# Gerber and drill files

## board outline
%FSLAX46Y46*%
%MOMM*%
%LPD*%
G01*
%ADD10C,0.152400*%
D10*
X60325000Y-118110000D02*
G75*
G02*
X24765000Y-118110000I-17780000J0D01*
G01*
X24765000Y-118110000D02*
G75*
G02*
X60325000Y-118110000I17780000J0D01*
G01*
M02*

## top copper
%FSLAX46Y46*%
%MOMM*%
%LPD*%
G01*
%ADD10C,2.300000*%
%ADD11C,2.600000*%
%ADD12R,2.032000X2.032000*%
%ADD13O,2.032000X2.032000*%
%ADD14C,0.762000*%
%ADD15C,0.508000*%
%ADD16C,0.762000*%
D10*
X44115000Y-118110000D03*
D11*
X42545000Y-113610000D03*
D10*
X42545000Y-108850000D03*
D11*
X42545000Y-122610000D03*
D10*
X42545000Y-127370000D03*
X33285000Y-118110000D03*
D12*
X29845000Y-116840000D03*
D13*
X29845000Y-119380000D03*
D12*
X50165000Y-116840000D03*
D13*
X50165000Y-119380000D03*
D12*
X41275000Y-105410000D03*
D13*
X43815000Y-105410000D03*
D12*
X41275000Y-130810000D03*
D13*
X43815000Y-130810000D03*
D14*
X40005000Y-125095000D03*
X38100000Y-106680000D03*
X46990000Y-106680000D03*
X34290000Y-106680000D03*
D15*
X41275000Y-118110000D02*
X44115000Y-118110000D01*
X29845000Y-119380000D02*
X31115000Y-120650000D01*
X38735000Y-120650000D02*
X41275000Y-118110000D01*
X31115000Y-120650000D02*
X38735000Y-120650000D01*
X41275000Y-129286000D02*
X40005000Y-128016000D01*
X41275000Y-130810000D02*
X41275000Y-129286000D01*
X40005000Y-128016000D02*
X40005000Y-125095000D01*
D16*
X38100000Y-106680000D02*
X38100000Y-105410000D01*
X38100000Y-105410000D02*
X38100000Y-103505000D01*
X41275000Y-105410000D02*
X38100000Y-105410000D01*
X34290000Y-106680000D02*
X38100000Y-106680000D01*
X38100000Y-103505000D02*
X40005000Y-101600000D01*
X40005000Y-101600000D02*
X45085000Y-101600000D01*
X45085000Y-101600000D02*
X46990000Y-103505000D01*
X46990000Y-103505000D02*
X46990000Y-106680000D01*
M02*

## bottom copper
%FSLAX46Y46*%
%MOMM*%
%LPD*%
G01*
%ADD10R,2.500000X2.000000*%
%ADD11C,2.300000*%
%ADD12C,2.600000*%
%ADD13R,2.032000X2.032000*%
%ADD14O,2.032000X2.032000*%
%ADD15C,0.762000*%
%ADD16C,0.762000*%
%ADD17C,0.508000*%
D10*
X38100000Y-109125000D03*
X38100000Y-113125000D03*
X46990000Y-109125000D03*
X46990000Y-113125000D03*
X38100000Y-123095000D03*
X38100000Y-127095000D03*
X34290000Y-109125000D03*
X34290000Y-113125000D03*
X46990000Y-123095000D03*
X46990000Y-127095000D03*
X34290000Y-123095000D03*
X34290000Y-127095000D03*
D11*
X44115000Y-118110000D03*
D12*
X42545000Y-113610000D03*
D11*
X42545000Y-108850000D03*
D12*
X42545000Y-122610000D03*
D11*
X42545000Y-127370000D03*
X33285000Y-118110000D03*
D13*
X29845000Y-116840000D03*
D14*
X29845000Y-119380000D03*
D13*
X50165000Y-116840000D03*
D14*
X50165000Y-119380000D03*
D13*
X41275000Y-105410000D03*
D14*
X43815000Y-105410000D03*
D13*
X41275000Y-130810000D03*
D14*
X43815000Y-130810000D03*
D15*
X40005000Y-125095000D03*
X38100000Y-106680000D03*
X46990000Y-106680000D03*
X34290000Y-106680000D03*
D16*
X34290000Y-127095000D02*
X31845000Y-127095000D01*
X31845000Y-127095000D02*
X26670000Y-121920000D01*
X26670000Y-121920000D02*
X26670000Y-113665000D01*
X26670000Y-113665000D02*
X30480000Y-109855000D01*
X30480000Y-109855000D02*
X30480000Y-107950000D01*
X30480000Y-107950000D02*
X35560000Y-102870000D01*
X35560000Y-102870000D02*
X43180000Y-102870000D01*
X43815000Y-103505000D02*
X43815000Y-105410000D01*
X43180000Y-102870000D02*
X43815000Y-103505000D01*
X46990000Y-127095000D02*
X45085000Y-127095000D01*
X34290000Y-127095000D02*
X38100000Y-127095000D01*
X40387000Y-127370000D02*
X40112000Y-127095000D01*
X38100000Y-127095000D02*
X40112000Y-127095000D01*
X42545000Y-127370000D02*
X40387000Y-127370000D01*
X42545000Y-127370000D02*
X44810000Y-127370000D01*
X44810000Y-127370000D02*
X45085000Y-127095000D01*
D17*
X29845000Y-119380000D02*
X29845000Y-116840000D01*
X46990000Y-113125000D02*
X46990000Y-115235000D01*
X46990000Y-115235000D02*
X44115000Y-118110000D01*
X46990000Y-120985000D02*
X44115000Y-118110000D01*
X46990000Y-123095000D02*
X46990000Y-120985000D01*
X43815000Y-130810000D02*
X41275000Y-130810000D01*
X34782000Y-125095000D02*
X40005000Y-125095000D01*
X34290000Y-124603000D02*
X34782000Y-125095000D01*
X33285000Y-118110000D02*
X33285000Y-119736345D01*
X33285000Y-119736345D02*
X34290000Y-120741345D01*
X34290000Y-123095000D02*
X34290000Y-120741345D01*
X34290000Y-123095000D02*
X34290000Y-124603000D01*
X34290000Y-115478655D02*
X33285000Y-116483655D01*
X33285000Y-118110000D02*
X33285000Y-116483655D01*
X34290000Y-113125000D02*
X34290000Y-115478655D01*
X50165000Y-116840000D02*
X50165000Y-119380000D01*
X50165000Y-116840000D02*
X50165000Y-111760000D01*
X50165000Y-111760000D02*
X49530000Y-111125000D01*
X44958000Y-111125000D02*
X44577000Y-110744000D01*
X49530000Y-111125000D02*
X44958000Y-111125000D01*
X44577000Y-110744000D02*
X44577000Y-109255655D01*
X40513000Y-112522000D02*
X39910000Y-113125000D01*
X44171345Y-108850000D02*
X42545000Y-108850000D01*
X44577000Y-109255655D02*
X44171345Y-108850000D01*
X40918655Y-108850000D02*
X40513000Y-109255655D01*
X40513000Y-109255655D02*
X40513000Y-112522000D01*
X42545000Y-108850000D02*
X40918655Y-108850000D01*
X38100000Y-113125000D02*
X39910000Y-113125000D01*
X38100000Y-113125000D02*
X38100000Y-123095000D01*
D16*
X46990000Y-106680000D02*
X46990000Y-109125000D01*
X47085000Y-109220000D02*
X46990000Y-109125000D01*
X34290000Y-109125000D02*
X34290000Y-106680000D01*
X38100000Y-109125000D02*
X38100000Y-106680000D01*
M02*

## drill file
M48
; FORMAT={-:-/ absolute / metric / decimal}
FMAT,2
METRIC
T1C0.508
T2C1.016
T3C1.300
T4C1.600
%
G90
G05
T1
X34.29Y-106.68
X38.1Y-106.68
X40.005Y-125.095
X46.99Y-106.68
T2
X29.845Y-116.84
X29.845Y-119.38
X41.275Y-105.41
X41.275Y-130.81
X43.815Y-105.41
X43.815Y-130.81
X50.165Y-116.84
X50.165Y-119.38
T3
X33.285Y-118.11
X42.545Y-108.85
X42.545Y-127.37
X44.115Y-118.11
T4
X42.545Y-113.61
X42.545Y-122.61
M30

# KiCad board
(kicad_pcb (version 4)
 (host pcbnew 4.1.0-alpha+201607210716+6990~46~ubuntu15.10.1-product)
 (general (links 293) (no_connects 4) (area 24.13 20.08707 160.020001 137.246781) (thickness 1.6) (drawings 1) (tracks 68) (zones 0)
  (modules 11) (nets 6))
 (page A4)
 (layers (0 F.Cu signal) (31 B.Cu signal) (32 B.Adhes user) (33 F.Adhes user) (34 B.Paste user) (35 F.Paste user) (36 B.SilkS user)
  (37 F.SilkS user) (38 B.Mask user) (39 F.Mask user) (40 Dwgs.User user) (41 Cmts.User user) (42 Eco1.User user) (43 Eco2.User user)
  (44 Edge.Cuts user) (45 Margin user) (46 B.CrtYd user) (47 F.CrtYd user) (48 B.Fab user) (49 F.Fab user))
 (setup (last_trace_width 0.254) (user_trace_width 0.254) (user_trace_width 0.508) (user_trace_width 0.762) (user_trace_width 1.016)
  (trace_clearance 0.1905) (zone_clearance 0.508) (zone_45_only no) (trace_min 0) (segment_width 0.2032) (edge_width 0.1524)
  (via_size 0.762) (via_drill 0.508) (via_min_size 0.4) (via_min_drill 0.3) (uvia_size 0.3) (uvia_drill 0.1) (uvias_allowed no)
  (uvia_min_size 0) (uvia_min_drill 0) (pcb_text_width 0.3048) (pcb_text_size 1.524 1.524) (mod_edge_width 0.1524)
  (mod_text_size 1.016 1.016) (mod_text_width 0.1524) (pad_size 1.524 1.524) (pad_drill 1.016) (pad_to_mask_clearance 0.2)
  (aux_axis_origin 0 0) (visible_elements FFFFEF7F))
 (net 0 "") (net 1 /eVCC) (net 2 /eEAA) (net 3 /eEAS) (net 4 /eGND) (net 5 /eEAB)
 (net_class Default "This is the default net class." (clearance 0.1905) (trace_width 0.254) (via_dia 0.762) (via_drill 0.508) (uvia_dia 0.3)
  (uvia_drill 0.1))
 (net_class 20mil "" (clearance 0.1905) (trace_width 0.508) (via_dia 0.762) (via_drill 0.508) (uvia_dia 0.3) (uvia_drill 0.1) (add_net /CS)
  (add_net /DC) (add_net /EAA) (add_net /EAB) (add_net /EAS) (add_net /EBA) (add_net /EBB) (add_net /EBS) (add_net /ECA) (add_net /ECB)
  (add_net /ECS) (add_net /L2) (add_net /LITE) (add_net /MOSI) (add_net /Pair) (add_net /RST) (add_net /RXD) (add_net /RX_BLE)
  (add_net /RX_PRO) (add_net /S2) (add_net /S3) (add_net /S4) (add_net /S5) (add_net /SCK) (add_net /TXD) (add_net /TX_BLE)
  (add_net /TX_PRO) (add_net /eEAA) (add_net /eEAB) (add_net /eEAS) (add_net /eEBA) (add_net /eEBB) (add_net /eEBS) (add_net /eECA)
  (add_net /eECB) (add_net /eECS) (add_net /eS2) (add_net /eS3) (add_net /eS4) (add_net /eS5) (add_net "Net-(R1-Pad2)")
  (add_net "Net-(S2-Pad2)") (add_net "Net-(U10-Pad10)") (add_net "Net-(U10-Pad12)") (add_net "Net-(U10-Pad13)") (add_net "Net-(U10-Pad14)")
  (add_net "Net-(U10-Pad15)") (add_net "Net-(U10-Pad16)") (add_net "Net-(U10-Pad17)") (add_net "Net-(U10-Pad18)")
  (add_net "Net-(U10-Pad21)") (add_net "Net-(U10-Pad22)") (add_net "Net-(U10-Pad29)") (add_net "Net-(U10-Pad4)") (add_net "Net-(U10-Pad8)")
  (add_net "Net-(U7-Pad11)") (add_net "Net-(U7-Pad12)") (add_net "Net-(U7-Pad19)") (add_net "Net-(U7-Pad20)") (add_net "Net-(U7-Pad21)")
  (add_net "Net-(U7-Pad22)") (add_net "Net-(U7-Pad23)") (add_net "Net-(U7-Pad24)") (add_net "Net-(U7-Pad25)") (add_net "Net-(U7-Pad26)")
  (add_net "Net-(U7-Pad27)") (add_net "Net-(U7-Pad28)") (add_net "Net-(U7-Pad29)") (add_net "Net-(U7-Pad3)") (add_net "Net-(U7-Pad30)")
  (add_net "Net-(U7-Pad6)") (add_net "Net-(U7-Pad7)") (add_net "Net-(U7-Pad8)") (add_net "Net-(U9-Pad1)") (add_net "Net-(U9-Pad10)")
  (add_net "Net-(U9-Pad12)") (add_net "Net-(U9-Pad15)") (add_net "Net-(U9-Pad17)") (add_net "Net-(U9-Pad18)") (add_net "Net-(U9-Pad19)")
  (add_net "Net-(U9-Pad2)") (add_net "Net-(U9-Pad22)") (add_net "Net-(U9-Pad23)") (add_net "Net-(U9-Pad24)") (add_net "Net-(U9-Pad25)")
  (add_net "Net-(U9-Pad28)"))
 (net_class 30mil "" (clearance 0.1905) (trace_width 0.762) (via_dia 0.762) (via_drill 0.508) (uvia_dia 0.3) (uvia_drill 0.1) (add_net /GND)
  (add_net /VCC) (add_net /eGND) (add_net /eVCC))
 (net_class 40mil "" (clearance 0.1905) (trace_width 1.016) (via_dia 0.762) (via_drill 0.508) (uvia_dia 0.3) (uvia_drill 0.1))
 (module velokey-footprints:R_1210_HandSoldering (layer B.Cu) (at 38.1 111.125 270)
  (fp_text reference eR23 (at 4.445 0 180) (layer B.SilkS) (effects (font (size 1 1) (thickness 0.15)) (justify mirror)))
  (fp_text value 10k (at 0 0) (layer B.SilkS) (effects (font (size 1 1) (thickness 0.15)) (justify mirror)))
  (pad 1 smd rect (at -2 0 270) (size 2 2.5) (layers B.Cu B.Paste B.Mask) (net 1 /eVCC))
  (pad 2 smd rect (at 2 0 270) (size 2 2.5) (layers B.Cu B.Paste B.Mask) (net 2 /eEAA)))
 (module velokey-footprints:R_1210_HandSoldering (layer B.Cu) (at 46.99 111.125 270)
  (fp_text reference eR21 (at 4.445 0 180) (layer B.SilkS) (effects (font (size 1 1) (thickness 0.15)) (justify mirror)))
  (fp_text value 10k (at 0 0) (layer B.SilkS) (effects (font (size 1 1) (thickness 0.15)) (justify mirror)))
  (pad 1 smd rect (at -2 0 270) (size 2 2.5) (layers B.Cu B.Paste B.Mask) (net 1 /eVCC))
  (pad 2 smd rect (at 2 0 270) (size 2 2.5) (layers B.Cu B.Paste B.Mask) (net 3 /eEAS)))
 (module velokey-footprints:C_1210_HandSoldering (layer B.Cu) (at 38.1 125.095 270)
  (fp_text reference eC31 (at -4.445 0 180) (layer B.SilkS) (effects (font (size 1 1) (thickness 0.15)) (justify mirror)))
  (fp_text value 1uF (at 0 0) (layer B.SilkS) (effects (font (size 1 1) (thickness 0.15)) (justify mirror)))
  (pad 1 smd rect (at -2 0 270) (size 2 2.5) (layers B.Cu B.Paste B.Mask) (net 2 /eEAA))
  (pad 2 smd rect (at 2 0 270) (size 2 2.5) (layers B.Cu B.Paste B.Mask) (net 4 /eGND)))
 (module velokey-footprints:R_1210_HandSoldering (layer B.Cu) (at 34.29 111.125 270)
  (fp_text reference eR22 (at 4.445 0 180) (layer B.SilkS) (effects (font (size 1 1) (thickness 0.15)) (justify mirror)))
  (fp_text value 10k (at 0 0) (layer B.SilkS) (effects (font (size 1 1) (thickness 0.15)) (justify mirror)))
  (pad 1 smd rect (at -2 0 270) (size 2 2.5) (layers B.Cu B.Paste B.Mask) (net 1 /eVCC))
  (pad 2 smd rect (at 2 0 270) (size 2 2.5) (layers B.Cu B.Paste B.Mask) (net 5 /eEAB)))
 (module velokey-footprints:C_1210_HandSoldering (layer B.Cu) (at 46.99 125.095 270)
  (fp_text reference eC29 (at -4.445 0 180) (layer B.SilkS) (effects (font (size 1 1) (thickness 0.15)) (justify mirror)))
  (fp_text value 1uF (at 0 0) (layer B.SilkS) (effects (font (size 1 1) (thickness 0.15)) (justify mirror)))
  (pad 1 smd rect (at -2 0 270) (size 2 2.5) (layers B.Cu B.Paste B.Mask) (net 3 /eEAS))
  (pad 2 smd rect (at 2 0 270) (size 2 2.5) (layers B.Cu B.Paste B.Mask) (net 4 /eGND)))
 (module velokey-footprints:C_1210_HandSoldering (layer B.Cu) (at 34.29 125.095 270)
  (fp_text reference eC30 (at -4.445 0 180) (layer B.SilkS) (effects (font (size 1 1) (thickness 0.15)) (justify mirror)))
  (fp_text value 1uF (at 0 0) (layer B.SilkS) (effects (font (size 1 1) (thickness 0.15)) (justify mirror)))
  (pad 1 smd rect (at -2 0 270) (size 2 2.5) (layers B.Cu B.Paste B.Mask) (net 5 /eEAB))
  (pad 2 smd rect (at 2 0 270) (size 2 2.5) (layers B.Cu B.Paste B.Mask) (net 4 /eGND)))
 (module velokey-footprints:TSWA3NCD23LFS (layer F.Cu) (at 42.545 118.11 270)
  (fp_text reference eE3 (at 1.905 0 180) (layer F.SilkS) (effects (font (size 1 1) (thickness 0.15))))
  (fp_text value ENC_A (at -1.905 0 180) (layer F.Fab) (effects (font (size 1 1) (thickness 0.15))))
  (pad 4 thru_hole circle (at 0 -1.57 270) (size 2.3 2.3) (drill 1.3) (layers *.Cu *.Mask F.SilkS) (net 3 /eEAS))
  (pad 5 thru_hole circle (at -4.5 0 270) (size 2.6 2.6) (drill 1.6) (layers *.Cu *.Mask F.SilkS))
  (pad 1 thru_hole circle (at -9.26 0 270) (size 2.3 2.3) (drill 1.3) (layers *.Cu *.Mask F.SilkS) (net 2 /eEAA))
  (pad 6 thru_hole circle (at 4.5 0 270) (size 2.6 2.6) (drill 1.6) (layers *.Cu *.Mask F.SilkS))
  (pad 2 thru_hole circle (at 9.26 0 270) (size 2.3 2.3) (drill 1.3) (layers *.Cu *.Mask F.SilkS) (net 4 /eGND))
  (pad 3 thru_hole circle (at 0 9.26 270) (size 2.3 2.3) (drill 1.3) (layers *.Cu *.Mask F.SilkS) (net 5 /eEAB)))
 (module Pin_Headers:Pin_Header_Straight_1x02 (layer F.Cu) (at 29.845 116.84)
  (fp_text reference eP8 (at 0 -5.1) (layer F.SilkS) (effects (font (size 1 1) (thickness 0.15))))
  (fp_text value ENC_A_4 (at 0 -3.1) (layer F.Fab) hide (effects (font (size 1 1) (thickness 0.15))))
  (pad 1 thru_hole rect (at 0 0) (size 2.032 2.032) (drill 1.016) (layers *.Cu *.Mask F.SilkS) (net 3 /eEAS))
  (pad 2 thru_hole oval (at 0 2.54) (size 2.032 2.032) (drill 1.016) (layers *.Cu *.Mask F.SilkS) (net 3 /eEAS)))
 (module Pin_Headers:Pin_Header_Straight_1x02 (layer F.Cu) (at 50.165 116.84)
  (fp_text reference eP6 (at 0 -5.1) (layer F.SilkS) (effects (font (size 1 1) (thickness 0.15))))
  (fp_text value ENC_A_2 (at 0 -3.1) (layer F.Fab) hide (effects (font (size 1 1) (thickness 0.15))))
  (pad 1 thru_hole rect (at 0 0) (size 2.032 2.032) (drill 1.016) (layers *.Cu *.Mask F.SilkS) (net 2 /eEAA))
  (pad 2 thru_hole oval (at 0 2.54) (size 2.032 2.032) (drill 1.016) (layers *.Cu *.Mask F.SilkS) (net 2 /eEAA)))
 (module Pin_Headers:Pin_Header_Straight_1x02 (layer F.Cu) (at 41.275 105.41 90)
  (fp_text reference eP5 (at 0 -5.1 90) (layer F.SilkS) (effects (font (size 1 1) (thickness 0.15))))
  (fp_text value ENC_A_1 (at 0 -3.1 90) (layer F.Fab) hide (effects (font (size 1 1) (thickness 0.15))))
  (pad 1 thru_hole rect (at 0 0 90) (size 2.032 2.032) (drill 1.016) (layers *.Cu *.Mask F.SilkS) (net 1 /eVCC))
  (pad 2 thru_hole oval (at 0 2.54 90) (size 2.032 2.032) (drill 1.016) (layers *.Cu *.Mask F.SilkS) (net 4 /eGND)))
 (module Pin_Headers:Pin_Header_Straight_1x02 (layer F.Cu) (at 41.275 130.81 90)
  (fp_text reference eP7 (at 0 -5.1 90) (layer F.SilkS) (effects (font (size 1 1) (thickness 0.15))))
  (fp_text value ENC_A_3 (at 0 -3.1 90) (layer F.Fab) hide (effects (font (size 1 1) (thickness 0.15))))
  (pad 1 thru_hole rect (at 0 0 90) (size 2.032 2.032) (drill 1.016) (layers *.Cu *.Mask F.SilkS) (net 5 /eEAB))
  (pad 2 thru_hole oval (at 0 2.54 90) (size 2.032 2.032) (drill 1.016) (layers *.Cu *.Mask F.SilkS) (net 5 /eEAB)))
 (gr_circle (center 42.545 118.11) (end 60.325 118.11) (layer Edge.Cuts) (width 0.1524))
 (segment (start 34.29 127.095) (end 31.845 127.095) (width 0.762) (layer B.Cu) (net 4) (status 10))
 (segment (start 31.845 127.095) (end 26.67 121.92) (width 0.762) (layer B.Cu) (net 4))
 (segment (start 26.67 121.92) (end 26.67 113.665) (width 0.762) (layer B.Cu) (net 4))
 (segment (start 26.67 113.665) (end 30.48 109.855) (width 0.762) (layer B.Cu) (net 4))
 (segment (start 30.48 109.855) (end 30.48 107.95) (width 0.762) (layer B.Cu) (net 4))
 (segment (start 30.48 107.95) (end 35.56 102.87) (width 0.762) (layer B.Cu) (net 4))
 (segment (start 35.56 102.87) (end 43.18 102.87) (width 0.762) (layer B.Cu) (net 4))
 (segment (start 43.815 103.505) (end 43.815 105.41) (width 0.762) (layer B.Cu) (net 4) (status 20))
 (segment (start 43.18 102.87) (end 43.815 103.505) (width 0.762) (layer B.Cu) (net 4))
 (segment (start 46.99 127.095) (end 45.085 127.095) (width 0.762) (layer B.Cu) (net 4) (status 10))
 (segment (start 34.29 127.095) (end 38.1 127.095) (width 0.762) (layer B.Cu) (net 4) (status 30))
 (segment (start 40.387 127.37) (end 40.112 127.095) (width 0.762) (layer B.Cu) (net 4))
 (segment (start 38.1 127.095) (end 40.112 127.095) (width 0.762) (layer B.Cu) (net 4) (status 10))
 (segment (start 42.545 127.37) (end 40.387 127.37) (width 0.762) (layer B.Cu) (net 4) (status 10))
 (segment (start 42.545 127.37) (end 44.81 127.37) (width 0.762) (layer B.Cu) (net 4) (status 10))
 (segment (start 44.81 127.37) (end 45.085 127.095) (width 0.762) (layer B.Cu) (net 4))
 (segment (start 29.845 119.38) (end 29.845 116.84) (width 0.508) (layer B.Cu) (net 3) (status 30))
 (segment (start 46.99 113.125) (end 46.99 115.235) (width 0.508) (layer B.Cu) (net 3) (status 10))
 (segment (start 46.99 115.235) (end 44.115 118.11) (width 0.508) (layer B.Cu) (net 3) (status 20))
 (segment (start 46.99 120.985) (end 44.115 118.11) (width 0.508) (layer B.Cu) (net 3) (status 20))
 (segment (start 46.99 123.095) (end 46.99 120.985) (width 0.508) (layer B.Cu) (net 3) (status 10))
 (segment (start 41.275 118.11) (end 44.115 118.11) (width 0.508) (layer F.Cu) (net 3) (status 20))
 (segment (start 29.845 119.38) (end 31.115 120.65) (width 0.508) (layer F.Cu) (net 3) (status 10))
 (segment (start 38.735 120.65) (end 41.275 118.11) (width 0.508) (layer F.Cu) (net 3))
 (segment (start 31.115 120.65) (end 38.735 120.65) (width 0.508) (layer F.Cu) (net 3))
 (segment (start 43.815 130.81) (end 41.275 130.81) (width 0.508) (layer B.Cu) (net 5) (status 30))
 (segment (start 34.782 125.095) (end 40.005 125.095) (width 0.508) (layer B.Cu) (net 5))
 (segment (start 34.29 124.603) (end 34.782 125.095) (width 0.508) (layer B.Cu) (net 5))
 (segment (start 33.285 118.11) (end 33.285 119.736345) (width 0.508) (layer B.Cu) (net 5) (status 10))
 (segment (start 33.285 119.736345) (end 34.29 120.741345) (width 0.508) (layer B.Cu) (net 5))
 (segment (start 34.29 123.095) (end 34.29 120.741345) (width 0.508) (layer B.Cu) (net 5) (status 10))
 (segment (start 34.29 123.095) (end 34.29 124.603) (width 0.508) (layer B.Cu) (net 5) (status 10))
 (segment (start 34.29 115.478655) (end 33.285 116.483655) (width 0.508) (layer B.Cu) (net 5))
 (segment (start 33.285 118.11) (end 33.285 116.483655) (width 0.508) (layer B.Cu) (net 5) (status 10))
 (segment (start 34.29 113.125) (end 34.29 115.478655) (width 0.508) (layer B.Cu) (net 5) (status 10))
 (segment (start 41.275 129.286) (end 40.005 128.016) (width 0.508) (layer F.Cu) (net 5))
 (segment (start 41.275 130.81) (end 41.275 129.286) (width 0.508) (layer F.Cu) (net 5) (status 10))
 (segment (start 40.005 128.016) (end 40.005 125.095) (width 0.508) (layer F.Cu) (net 5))
 (via (at 40.005 125.095) (size 0.762) (drill 0.508) (layers F.Cu B.Cu) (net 5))
 (segment (start 50.165 116.84) (end 50.165 119.38) (width 0.508) (layer B.Cu) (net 2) (status 30))
 (segment (start 50.165 116.84) (end 50.165 111.76) (width 0.508) (layer B.Cu) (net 2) (status 10))
 (segment (start 50.165 111.76) (end 49.53 111.125) (width 0.508) (layer B.Cu) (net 2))
 (segment (start 44.958 111.125) (end 44.577 110.744) (width 0.508) (layer B.Cu) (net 2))
 (segment (start 49.53 111.125) (end 44.958 111.125) (width 0.508) (layer B.Cu) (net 2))
 (segment (start 44.577 110.744) (end 44.577 109.255655) (width 0.508) (layer B.Cu) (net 2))
 (segment (start 40.513 112.522) (end 39.91 113.125) (width 0.508) (layer B.Cu) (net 2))
 (segment (start 44.171345 108.85) (end 42.545 108.85) (width 0.508) (layer B.Cu) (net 2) (status 20))
 (segment (start 44.577 109.255655) (end 44.171345 108.85) (width 0.508) (layer B.Cu) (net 2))
 (segment (start 40.918655 108.85) (end 40.513 109.255655) (width 0.508) (layer B.Cu) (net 2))
 (segment (start 40.513 109.255655) (end 40.513 112.522) (width 0.508) (layer B.Cu) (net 2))
 (segment (start 42.545 108.85) (end 40.918655 108.85) (width 0.508) (layer B.Cu) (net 2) (status 10))
 (segment (start 38.1 113.125) (end 39.91 113.125) (width 0.508) (layer B.Cu) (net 2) (status 10))
 (segment (start 38.1 113.125) (end 38.1 123.095) (width 0.508) (layer B.Cu) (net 2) (status 30))
 (segment (start 38.1 106.68) (end 38.1 105.41) (width 0.762) (layer F.Cu) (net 1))
 (segment (start 38.1 105.41) (end 38.1 103.505) (width 0.762) (layer F.Cu) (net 1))
 (segment (start 41.275 105.41) (end 38.1 105.41) (width 0.762) (layer F.Cu) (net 1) (status 10))
 (segment (start 46.99 106.68) (end 46.99 109.125) (width 0.762) (layer B.Cu) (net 1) (status 20))
 (segment (start 47.085 109.22) (end 46.99 109.125) (width 0.762) (layer B.Cu) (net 1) (status 30))
 (segment (start 34.29 109.125) (end 34.29 106.68) (width 0.762) (layer B.Cu) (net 1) (status 10))
 (segment (start 38.1 109.125) (end 38.1 106.68) (width 0.762) (layer B.Cu) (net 1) (status 10))
 (segment (start 34.29 106.68) (end 38.1 106.68) (width 0.762) (layer F.Cu) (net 1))
 (segment (start 38.1 103.505) (end 40.005 101.6) (width 0.762) (layer F.Cu) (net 1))
 (segment (start 40.005 101.6) (end 45.085 101.6) (width 0.762) (layer F.Cu) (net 1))
 (segment (start 45.085 101.6) (end 46.99 103.505) (width 0.762) (layer F.Cu) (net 1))
 (segment (start 46.99 103.505) (end 46.99 106.68) (width 0.762) (layer F.Cu) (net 1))
 (via (at 38.1 106.68) (size 0.762) (drill 0.508) (layers F.Cu B.Cu) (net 1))
 (via (at 46.99 106.68) (size 0.762) (drill 0.508) (layers F.Cu B.Cu) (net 1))
 (via (at 34.29 106.68) (size 0.762) (drill 0.508) (layers F.Cu B.Cu) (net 1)))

